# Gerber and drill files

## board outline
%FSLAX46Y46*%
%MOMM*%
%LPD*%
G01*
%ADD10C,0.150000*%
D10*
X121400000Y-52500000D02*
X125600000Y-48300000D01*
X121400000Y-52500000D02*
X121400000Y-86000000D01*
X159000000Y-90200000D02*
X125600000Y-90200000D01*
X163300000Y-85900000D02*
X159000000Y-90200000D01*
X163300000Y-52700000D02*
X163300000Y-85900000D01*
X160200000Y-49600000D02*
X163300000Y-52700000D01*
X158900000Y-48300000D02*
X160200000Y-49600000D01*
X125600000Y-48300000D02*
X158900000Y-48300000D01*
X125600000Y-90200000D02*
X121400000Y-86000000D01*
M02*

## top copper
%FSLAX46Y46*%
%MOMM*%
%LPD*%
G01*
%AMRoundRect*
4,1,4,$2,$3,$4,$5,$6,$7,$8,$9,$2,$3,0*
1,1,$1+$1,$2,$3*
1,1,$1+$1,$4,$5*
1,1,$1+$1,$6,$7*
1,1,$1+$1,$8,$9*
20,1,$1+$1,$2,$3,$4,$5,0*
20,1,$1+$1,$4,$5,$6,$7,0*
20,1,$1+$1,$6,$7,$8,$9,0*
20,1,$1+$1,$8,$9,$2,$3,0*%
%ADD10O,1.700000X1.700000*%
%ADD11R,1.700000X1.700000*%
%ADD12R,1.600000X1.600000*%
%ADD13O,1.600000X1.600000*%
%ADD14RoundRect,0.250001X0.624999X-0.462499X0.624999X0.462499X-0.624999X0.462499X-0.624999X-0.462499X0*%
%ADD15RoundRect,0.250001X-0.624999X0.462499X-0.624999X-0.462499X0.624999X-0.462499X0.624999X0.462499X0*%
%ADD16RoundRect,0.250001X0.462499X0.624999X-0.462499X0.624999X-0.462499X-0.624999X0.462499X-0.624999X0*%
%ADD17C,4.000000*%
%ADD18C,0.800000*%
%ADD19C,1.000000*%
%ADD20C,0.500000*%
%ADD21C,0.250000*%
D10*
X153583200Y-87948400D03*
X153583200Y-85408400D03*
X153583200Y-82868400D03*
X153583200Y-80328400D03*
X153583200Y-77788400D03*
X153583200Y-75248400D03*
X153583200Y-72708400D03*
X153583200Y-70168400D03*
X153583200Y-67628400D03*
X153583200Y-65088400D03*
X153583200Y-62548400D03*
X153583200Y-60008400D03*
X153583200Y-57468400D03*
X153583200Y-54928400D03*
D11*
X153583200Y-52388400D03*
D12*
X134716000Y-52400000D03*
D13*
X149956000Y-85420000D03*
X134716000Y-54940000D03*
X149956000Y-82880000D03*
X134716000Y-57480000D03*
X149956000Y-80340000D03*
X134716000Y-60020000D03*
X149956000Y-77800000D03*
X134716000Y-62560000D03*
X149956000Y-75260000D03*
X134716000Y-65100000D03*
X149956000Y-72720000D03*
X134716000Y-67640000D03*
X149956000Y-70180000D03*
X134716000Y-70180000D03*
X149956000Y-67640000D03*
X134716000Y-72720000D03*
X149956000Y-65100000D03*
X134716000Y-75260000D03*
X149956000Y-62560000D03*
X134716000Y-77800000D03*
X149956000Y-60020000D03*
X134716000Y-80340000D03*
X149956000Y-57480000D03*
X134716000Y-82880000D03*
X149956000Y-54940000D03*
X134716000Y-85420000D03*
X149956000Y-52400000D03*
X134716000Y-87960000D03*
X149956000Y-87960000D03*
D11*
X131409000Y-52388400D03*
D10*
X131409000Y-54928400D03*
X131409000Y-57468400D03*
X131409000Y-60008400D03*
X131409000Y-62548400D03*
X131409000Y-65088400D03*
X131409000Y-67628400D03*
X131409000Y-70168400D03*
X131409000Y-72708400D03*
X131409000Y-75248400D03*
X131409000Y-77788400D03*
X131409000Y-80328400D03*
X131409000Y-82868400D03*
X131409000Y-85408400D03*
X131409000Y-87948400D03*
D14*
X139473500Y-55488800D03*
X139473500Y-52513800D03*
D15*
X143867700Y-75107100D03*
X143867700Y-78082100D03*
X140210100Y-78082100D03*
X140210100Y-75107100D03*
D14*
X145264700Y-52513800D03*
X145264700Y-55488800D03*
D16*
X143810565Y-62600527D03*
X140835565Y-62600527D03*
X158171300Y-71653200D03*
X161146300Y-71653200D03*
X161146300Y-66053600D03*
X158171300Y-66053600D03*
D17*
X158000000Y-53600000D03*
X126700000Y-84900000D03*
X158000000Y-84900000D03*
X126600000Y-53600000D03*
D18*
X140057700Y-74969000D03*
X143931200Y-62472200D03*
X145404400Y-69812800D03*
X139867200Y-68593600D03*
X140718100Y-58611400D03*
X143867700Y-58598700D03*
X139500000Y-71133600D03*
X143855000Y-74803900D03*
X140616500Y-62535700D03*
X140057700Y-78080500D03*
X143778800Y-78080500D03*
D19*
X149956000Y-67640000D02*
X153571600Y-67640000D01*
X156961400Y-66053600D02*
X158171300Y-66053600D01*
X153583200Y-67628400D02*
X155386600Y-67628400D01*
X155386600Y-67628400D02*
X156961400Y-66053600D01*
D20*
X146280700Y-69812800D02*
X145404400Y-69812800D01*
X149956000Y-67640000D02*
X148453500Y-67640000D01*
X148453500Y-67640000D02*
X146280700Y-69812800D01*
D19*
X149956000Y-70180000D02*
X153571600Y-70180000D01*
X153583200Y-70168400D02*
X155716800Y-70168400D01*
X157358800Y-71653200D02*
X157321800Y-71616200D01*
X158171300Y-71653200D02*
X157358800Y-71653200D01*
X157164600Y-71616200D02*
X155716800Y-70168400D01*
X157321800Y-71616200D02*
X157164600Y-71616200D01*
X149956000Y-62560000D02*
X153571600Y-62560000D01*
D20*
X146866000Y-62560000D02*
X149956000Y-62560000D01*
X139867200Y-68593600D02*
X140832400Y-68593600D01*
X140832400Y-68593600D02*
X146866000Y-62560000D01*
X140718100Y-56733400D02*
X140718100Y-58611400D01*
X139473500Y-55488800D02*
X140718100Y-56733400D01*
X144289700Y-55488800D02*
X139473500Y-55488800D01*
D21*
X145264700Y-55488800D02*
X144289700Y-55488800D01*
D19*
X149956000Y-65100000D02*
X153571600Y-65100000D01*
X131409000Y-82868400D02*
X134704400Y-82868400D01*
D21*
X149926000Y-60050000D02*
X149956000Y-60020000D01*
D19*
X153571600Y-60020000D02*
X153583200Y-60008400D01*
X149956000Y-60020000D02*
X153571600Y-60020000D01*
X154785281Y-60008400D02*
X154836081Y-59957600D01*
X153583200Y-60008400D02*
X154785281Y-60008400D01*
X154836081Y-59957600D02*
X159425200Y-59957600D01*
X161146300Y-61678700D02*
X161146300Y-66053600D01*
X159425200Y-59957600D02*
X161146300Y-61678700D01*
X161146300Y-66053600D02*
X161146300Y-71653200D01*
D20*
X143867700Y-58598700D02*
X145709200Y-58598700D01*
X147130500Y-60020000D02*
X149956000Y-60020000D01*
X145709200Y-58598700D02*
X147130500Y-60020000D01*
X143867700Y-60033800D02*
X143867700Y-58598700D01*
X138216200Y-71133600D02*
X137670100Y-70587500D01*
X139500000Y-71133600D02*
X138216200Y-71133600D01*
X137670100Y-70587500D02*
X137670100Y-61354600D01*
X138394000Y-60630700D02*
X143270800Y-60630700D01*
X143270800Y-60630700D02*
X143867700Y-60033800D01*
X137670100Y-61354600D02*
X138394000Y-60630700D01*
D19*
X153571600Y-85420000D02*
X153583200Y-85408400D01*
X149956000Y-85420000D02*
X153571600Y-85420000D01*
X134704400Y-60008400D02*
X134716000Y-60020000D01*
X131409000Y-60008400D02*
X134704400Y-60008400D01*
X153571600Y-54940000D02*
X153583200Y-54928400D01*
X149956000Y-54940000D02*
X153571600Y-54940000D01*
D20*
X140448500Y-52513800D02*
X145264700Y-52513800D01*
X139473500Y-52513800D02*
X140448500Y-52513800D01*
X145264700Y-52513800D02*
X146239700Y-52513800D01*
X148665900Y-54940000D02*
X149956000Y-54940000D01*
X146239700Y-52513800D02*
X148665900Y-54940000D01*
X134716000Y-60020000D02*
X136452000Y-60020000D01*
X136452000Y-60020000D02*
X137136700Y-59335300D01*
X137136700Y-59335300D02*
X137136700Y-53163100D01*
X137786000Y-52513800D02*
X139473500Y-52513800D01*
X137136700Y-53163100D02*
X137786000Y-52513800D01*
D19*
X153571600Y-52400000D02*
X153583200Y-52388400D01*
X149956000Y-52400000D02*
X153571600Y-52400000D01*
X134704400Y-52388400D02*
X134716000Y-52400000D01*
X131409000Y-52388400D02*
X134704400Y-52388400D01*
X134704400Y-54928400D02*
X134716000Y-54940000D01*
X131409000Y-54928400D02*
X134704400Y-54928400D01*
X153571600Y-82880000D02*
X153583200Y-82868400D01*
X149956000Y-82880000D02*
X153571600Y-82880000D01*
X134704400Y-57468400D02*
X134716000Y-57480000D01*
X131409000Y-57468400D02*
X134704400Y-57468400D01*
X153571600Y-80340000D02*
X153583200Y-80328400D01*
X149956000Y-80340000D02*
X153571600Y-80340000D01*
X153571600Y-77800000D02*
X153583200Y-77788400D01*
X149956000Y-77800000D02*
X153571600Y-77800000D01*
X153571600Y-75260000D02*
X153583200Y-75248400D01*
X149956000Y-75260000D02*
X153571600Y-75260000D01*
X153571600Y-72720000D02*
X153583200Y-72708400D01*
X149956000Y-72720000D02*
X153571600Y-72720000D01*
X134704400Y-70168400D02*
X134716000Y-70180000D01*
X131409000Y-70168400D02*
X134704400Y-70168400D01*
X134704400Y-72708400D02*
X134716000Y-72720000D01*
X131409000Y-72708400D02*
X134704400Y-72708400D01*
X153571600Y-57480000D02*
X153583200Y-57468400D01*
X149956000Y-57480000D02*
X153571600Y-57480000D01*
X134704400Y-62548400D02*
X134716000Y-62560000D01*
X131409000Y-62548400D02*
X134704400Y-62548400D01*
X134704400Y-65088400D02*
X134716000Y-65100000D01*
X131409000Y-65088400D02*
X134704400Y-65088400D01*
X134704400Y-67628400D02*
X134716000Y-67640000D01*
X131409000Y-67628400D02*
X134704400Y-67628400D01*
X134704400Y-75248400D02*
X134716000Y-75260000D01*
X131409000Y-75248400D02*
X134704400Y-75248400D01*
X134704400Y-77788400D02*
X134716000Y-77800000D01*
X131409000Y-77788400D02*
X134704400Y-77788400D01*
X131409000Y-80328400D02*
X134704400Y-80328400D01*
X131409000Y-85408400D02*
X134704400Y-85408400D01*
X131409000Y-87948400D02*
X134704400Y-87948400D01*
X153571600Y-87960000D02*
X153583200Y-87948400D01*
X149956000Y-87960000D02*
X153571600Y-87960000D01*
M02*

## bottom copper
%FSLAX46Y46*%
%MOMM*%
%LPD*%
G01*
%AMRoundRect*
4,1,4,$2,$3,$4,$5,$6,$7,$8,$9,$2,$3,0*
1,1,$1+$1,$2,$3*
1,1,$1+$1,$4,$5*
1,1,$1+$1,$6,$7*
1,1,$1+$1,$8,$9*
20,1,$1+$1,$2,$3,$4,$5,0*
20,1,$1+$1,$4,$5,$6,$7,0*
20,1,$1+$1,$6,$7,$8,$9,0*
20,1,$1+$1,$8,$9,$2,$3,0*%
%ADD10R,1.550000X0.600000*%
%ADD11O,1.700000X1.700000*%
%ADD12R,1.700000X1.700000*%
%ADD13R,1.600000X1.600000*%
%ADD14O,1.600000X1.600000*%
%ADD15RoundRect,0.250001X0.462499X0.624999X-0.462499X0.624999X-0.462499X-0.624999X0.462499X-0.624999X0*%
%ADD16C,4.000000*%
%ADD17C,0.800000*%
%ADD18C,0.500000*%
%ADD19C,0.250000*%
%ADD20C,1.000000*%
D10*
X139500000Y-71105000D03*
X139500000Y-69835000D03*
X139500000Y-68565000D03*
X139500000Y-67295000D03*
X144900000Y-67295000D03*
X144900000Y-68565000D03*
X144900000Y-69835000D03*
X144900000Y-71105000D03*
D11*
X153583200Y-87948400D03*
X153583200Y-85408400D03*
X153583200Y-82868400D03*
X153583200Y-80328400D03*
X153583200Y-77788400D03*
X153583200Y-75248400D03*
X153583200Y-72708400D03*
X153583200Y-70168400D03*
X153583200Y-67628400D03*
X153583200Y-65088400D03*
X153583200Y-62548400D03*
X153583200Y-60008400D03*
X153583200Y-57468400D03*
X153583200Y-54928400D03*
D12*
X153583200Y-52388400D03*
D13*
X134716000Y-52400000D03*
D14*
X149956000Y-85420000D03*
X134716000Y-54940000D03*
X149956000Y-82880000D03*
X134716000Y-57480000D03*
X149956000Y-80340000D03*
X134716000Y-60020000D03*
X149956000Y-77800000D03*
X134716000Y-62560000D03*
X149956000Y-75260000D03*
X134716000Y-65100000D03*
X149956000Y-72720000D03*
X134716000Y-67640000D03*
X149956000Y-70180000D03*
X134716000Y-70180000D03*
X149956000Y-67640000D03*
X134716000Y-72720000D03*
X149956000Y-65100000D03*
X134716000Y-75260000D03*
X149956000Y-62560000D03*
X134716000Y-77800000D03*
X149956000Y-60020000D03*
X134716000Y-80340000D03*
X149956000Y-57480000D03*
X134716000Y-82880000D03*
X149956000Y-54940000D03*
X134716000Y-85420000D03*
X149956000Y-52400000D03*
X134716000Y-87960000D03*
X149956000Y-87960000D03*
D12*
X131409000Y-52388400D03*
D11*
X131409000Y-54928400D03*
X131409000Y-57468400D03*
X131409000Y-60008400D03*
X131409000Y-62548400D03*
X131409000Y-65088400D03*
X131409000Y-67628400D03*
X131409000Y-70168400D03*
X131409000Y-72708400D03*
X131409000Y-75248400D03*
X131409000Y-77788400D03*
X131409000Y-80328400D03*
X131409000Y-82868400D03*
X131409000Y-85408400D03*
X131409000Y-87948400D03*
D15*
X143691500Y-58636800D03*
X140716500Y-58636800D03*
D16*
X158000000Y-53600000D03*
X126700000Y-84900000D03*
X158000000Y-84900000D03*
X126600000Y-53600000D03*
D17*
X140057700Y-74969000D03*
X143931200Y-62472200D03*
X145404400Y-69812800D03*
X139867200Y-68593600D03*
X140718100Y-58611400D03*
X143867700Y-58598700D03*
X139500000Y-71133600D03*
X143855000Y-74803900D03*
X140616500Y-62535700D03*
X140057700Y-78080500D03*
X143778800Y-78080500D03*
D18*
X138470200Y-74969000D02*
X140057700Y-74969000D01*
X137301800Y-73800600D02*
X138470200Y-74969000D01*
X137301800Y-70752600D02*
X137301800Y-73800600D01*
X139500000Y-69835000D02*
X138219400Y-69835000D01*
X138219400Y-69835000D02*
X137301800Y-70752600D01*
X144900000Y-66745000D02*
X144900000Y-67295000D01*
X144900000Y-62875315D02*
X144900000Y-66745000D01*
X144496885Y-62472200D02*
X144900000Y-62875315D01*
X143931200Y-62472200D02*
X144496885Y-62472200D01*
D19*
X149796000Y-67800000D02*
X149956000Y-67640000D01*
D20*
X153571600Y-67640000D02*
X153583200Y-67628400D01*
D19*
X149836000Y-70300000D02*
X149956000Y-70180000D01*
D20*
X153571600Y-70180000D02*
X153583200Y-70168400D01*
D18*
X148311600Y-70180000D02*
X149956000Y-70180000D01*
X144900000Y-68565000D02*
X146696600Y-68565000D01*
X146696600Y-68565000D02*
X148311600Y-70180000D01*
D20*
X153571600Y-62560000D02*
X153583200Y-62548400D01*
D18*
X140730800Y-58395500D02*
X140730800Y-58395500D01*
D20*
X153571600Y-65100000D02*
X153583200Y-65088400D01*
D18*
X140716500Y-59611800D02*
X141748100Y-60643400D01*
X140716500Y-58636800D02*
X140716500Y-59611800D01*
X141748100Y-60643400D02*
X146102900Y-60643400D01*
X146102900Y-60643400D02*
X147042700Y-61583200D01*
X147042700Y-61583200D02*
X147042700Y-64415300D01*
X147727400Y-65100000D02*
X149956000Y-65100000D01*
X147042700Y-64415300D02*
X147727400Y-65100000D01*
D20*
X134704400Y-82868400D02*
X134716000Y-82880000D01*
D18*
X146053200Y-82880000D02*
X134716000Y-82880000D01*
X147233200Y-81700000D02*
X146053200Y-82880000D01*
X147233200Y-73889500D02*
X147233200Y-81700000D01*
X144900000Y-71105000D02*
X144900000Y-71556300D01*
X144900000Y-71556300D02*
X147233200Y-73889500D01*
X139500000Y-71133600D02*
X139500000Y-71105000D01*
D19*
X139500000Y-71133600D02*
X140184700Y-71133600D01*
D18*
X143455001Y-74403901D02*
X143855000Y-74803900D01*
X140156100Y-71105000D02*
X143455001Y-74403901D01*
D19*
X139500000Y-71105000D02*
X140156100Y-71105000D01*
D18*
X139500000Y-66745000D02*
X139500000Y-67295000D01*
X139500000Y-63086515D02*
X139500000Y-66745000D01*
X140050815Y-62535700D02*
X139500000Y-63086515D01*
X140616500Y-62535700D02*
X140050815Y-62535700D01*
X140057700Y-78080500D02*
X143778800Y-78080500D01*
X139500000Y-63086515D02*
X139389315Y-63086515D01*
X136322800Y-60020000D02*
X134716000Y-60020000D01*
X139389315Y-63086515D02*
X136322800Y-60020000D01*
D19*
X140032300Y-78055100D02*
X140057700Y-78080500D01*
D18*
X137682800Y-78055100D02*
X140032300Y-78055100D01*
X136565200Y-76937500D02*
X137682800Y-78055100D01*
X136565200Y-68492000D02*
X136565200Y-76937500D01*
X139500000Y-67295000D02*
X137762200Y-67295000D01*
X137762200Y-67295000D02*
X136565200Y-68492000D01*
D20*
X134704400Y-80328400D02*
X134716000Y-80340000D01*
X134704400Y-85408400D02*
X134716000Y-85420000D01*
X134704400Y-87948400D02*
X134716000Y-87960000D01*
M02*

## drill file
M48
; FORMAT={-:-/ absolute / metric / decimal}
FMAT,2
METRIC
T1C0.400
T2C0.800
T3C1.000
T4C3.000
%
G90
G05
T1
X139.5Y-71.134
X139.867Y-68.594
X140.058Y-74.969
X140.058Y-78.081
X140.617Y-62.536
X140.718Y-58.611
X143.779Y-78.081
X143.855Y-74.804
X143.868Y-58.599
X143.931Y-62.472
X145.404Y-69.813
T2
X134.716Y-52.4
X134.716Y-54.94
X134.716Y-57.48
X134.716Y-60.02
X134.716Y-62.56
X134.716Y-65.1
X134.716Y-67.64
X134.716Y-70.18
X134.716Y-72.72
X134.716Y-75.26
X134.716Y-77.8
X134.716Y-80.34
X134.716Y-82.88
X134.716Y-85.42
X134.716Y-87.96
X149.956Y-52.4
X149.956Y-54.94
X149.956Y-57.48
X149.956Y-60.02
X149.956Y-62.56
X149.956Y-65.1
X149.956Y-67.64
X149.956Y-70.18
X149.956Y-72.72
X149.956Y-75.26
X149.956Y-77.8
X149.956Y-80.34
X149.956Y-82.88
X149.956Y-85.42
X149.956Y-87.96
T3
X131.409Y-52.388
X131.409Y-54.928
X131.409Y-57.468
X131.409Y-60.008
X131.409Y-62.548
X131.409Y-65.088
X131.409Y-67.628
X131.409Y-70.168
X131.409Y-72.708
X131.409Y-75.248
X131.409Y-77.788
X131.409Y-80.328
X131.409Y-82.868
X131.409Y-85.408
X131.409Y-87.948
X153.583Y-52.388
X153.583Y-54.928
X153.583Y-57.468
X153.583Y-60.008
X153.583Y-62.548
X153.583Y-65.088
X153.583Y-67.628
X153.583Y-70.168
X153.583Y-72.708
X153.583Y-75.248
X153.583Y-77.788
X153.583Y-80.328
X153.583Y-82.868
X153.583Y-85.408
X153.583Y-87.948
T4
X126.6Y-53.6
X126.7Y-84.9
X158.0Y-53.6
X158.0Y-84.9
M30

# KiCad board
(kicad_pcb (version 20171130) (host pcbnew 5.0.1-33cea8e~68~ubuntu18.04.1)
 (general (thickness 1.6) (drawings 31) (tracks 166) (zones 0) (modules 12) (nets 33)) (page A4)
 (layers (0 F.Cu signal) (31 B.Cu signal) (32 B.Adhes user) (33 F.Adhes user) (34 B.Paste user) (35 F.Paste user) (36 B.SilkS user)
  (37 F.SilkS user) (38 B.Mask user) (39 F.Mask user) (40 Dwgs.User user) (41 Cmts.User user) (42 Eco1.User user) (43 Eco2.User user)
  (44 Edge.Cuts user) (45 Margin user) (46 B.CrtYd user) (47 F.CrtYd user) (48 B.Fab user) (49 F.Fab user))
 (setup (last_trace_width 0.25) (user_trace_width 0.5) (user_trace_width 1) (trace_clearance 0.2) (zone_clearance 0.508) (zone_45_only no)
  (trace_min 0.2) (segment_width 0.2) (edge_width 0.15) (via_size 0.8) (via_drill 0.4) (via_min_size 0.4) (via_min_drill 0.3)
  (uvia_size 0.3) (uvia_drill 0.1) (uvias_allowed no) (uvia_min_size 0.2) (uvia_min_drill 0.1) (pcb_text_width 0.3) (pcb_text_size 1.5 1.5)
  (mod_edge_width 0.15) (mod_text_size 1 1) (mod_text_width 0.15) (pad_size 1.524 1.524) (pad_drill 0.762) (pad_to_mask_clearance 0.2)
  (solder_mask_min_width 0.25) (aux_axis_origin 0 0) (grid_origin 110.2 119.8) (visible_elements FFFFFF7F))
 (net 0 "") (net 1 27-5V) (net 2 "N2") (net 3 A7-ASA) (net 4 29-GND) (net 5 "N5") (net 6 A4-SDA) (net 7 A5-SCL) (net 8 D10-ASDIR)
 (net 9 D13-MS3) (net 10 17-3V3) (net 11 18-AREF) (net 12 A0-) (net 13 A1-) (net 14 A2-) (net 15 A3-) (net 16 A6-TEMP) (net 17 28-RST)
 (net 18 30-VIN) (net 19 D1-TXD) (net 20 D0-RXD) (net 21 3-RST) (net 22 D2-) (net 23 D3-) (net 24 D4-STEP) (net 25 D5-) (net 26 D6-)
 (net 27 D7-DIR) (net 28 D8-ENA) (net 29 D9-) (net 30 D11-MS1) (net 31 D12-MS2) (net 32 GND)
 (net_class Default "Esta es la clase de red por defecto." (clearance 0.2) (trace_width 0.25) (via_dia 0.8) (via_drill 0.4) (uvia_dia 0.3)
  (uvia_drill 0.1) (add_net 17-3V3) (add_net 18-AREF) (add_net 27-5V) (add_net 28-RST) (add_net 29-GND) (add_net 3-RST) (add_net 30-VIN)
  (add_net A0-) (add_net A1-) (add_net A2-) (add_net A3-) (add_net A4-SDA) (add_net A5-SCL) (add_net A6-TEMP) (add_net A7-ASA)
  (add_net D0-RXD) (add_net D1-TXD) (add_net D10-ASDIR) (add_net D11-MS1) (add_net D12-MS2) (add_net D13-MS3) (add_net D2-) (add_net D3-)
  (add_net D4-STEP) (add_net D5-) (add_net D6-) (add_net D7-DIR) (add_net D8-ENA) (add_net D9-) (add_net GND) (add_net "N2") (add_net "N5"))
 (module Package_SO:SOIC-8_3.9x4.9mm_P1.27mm (layer B.Cu) (at 142.2 69.2)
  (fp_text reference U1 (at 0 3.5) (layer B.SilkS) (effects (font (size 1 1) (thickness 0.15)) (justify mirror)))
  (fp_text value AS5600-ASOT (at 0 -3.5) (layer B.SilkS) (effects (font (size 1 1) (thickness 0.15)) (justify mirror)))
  (pad 1 smd rect (at -2.7 1.905) (size 1.55 0.6) (layers B.Cu B.Paste B.Mask) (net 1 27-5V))
  (pad 2 smd rect (at -2.7 0.635) (size 1.55 0.6) (layers B.Cu B.Paste B.Mask) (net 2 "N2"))
  (pad 3 smd rect (at -2.7 -0.635) (size 1.55 0.6) (layers B.Cu B.Paste B.Mask) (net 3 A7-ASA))
  (pad 4 smd rect (at -2.7 -1.905) (size 1.55 0.6) (layers B.Cu B.Paste B.Mask) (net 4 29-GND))
  (pad 5 smd rect (at 2.7 -1.905) (size 1.55 0.6) (layers B.Cu B.Paste B.Mask) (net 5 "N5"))
  (pad 6 smd rect (at 2.7 -0.635) (size 1.55 0.6) (layers B.Cu B.Paste B.Mask) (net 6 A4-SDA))
  (pad 7 smd rect (at 2.7 0.635) (size 1.55 0.6) (layers B.Cu B.Paste B.Mask) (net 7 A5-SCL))
  (pad 8 smd rect (at 2.7 1.905) (size 1.55 0.6) (layers B.Cu B.Paste B.Mask) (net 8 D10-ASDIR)))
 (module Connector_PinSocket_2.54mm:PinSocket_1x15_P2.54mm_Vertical (layer F.Cu) (at 153.5832 52.3884)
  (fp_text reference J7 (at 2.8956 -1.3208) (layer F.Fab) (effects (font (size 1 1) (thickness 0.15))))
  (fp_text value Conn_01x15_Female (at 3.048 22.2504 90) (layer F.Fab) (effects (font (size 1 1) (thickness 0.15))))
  (pad 15 thru_hole oval (at 0 35.56) (size 1.7 1.7) (drill 1) (layers *.Cu *.Mask) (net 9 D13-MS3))
  (pad 14 thru_hole oval (at 0 33.02) (size 1.7 1.7) (drill 1) (layers *.Cu *.Mask) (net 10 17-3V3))
  (pad 13 thru_hole oval (at 0 30.48) (size 1.7 1.7) (drill 1) (layers *.Cu *.Mask) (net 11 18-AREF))
  (pad 12 thru_hole oval (at 0 27.94) (size 1.7 1.7) (drill 1) (layers *.Cu *.Mask) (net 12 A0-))
  (pad 11 thru_hole oval (at 0 25.4) (size 1.7 1.7) (drill 1) (layers *.Cu *.Mask) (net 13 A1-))
  (pad 10 thru_hole oval (at 0 22.86) (size 1.7 1.7) (drill 1) (layers *.Cu *.Mask) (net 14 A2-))
  (pad 9 thru_hole oval (at 0 20.32) (size 1.7 1.7) (drill 1) (layers *.Cu *.Mask) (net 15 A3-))
  (pad 8 thru_hole oval (at 0 17.78) (size 1.7 1.7) (drill 1) (layers *.Cu *.Mask) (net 6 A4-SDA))
  (pad 7 thru_hole oval (at 0 15.24) (size 1.7 1.7) (drill 1) (layers *.Cu *.Mask) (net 7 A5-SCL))
  (pad 6 thru_hole oval (at 0 12.7) (size 1.7 1.7) (drill 1) (layers *.Cu *.Mask) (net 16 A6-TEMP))
  (pad 5 thru_hole oval (at 0 10.16) (size 1.7 1.7) (drill 1) (layers *.Cu *.Mask) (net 3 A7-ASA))
  (pad 4 thru_hole oval (at 0 7.62) (size 1.7 1.7) (drill 1) (layers *.Cu *.Mask) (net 1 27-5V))
  (pad 3 thru_hole oval (at 0 5.08) (size 1.7 1.7) (drill 1) (layers *.Cu *.Mask) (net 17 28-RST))
  (pad 2 thru_hole oval (at 0 2.54) (size 1.7 1.7) (drill 1) (layers *.Cu *.Mask) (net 4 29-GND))
  (pad 1 thru_hole rect (at 0 0) (size 1.7 1.7) (drill 1) (layers *.Cu *.Mask) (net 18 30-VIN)))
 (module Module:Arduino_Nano (layer F.Cu) (at 134.716 52.4)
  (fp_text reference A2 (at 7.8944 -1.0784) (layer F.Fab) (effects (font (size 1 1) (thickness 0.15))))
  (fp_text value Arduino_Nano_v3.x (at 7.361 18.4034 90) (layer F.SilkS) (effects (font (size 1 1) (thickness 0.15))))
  (pad 1 thru_hole rect (at 0 0) (size 1.6 1.6) (drill 0.8) (layers *.Cu *.Mask) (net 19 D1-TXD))
  (pad 17 thru_hole oval (at 15.24 33.02) (size 1.6 1.6) (drill 0.8) (layers *.Cu *.Mask) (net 10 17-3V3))
  (pad 2 thru_hole oval (at 0 2.54) (size 1.6 1.6) (drill 0.8) (layers *.Cu *.Mask) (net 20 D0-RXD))
  (pad 18 thru_hole oval (at 15.24 30.48) (size 1.6 1.6) (drill 0.8) (layers *.Cu *.Mask) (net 11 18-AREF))
  (pad 3 thru_hole oval (at 0 5.08) (size 1.6 1.6) (drill 0.8) (layers *.Cu *.Mask) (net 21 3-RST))
  (pad 19 thru_hole oval (at 15.24 27.94) (size 1.6 1.6) (drill 0.8) (layers *.Cu *.Mask) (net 12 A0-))
  (pad 4 thru_hole oval (at 0 7.62) (size 1.6 1.6) (drill 0.8) (layers *.Cu *.Mask) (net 4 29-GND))
  (pad 20 thru_hole oval (at 15.24 25.4) (size 1.6 1.6) (drill 0.8) (layers *.Cu *.Mask) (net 13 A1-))
  (pad 5 thru_hole oval (at 0 10.16) (size 1.6 1.6) (drill 0.8) (layers *.Cu *.Mask) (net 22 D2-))
  (pad 21 thru_hole oval (at 15.24 22.86) (size 1.6 1.6) (drill 0.8) (layers *.Cu *.Mask) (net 14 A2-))
  (pad 6 thru_hole oval (at 0 12.7) (size 1.6 1.6) (drill 0.8) (layers *.Cu *.Mask) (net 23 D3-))
  (pad 22 thru_hole oval (at 15.24 20.32) (size 1.6 1.6) (drill 0.8) (layers *.Cu *.Mask) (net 15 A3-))
  (pad 7 thru_hole oval (at 0 15.24) (size 1.6 1.6) (drill 0.8) (layers *.Cu *.Mask) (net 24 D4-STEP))
  (pad 23 thru_hole oval (at 15.24 17.78) (size 1.6 1.6) (drill 0.8) (layers *.Cu *.Mask) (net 6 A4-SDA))
  (pad 8 thru_hole oval (at 0 17.78) (size 1.6 1.6) (drill 0.8) (layers *.Cu *.Mask) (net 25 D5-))
  (pad 24 thru_hole oval (at 15.24 15.24) (size 1.6 1.6) (drill 0.8) (layers *.Cu *.Mask) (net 7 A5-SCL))
  (pad 9 thru_hole oval (at 0 20.32) (size 1.6 1.6) (drill 0.8) (layers *.Cu *.Mask) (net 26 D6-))
  (pad 25 thru_hole oval (at 15.24 12.7) (size 1.6 1.6) (drill 0.8) (layers *.Cu *.Mask) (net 16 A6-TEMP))
  (pad 10 thru_hole oval (at 0 22.86) (size 1.6 1.6) (drill 0.8) (layers *.Cu *.Mask) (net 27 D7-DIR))
  (pad 26 thru_hole oval (at 15.24 10.16) (size 1.6 1.6) (drill 0.8) (layers *.Cu *.Mask) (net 3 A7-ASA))
  (pad 11 thru_hole oval (at 0 25.4) (size 1.6 1.6) (drill 0.8) (layers *.Cu *.Mask) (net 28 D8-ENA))
  (pad 27 thru_hole oval (at 15.24 7.62) (size 1.6 1.6) (drill 0.8) (layers *.Cu *.Mask) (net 1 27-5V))
  (pad 12 thru_hole oval (at 0 27.94) (size 1.6 1.6) (drill 0.8) (layers *.Cu *.Mask) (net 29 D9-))
  (pad 28 thru_hole oval (at 15.24 5.08) (size 1.6 1.6) (drill 0.8) (layers *.Cu *.Mask) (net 17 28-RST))
  (pad 13 thru_hole oval (at 0 30.48) (size 1.6 1.6) (drill 0.8) (layers *.Cu *.Mask) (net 8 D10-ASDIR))
  (pad 29 thru_hole oval (at 15.24 2.54) (size 1.6 1.6) (drill 0.8) (layers *.Cu *.Mask) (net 4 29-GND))
  (pad 14 thru_hole oval (at 0 33.02) (size 1.6 1.6) (drill 0.8) (layers *.Cu *.Mask) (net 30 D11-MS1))
  (pad 30 thru_hole oval (at 15.24 0) (size 1.6 1.6) (drill 0.8) (layers *.Cu *.Mask) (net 18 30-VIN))
  (pad 15 thru_hole oval (at 0 35.56) (size 1.6 1.6) (drill 0.8) (layers *.Cu *.Mask) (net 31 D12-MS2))
  (pad 16 thru_hole oval (at 15.24 35.56) (size 1.6 1.6) (drill 0.8) (layers *.Cu *.Mask) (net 9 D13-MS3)))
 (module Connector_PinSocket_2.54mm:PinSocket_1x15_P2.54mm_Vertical (layer F.Cu) (at 131.409 52.3884)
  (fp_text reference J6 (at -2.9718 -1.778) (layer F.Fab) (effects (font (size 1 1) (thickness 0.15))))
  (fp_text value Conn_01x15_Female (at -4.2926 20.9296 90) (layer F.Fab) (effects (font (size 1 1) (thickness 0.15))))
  (pad 1 thru_hole rect (at 0 0) (size 1.7 1.7) (drill 1) (layers *.Cu *.Mask) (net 19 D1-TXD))
  (pad 2 thru_hole oval (at 0 2.54) (size 1.7 1.7) (drill 1) (layers *.Cu *.Mask) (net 20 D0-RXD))
  (pad 3 thru_hole oval (at 0 5.08) (size 1.7 1.7) (drill 1) (layers *.Cu *.Mask) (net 21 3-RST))
  (pad 4 thru_hole oval (at 0 7.62) (size 1.7 1.7) (drill 1) (layers *.Cu *.Mask) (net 4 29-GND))
  (pad 5 thru_hole oval (at 0 10.16) (size 1.7 1.7) (drill 1) (layers *.Cu *.Mask) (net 22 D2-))
  (pad 6 thru_hole oval (at 0 12.7) (size 1.7 1.7) (drill 1) (layers *.Cu *.Mask) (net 23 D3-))
  (pad 7 thru_hole oval (at 0 15.24) (size 1.7 1.7) (drill 1) (layers *.Cu *.Mask) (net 24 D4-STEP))
  (pad 8 thru_hole oval (at 0 17.78) (size 1.7 1.7) (drill 1) (layers *.Cu *.Mask) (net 25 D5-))
  (pad 9 thru_hole oval (at 0 20.32) (size 1.7 1.7) (drill 1) (layers *.Cu *.Mask) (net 26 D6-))
  (pad 10 thru_hole oval (at 0 22.86) (size 1.7 1.7) (drill 1) (layers *.Cu *.Mask) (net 27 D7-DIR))
  (pad 11 thru_hole oval (at 0 25.4) (size 1.7 1.7) (drill 1) (layers *.Cu *.Mask) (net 28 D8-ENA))
  (pad 12 thru_hole oval (at 0 27.94) (size 1.7 1.7) (drill 1) (layers *.Cu *.Mask) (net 29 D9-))
  (pad 13 thru_hole oval (at 0 30.48) (size 1.7 1.7) (drill 1) (layers *.Cu *.Mask) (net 8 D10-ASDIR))
  (pad 14 thru_hole oval (at 0 33.02) (size 1.7 1.7) (drill 1) (layers *.Cu *.Mask) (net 30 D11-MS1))
  (pad 15 thru_hole oval (at 0 35.56) (size 1.7 1.7) (drill 1) (layers *.Cu *.Mask) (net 31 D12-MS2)))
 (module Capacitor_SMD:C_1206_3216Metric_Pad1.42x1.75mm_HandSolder (layer F.Cu) (at 139.4735 54.0013 90)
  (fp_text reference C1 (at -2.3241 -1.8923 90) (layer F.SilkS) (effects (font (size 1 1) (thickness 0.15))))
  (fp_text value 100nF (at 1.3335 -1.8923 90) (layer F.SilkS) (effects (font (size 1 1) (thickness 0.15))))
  (pad 1 smd roundrect (at -1.4875 0 90) (size 1.425 1.75) (layers F.Cu F.Paste F.Mask) (roundrect_rratio 0.175439) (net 16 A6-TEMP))
  (pad 2 smd roundrect (at 1.4875 0 90) (size 1.425 1.75) (layers F.Cu F.Paste F.Mask) (roundrect_rratio 0.175439) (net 4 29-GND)))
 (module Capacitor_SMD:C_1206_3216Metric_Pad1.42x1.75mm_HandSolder (layer F.Cu) (at 143.8677 76.5946 270)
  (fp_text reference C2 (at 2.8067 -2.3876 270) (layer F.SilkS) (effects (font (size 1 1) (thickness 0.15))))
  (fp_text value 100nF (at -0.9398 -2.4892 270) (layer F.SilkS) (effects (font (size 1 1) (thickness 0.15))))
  (pad 1 smd roundrect (at -1.4875 0 270) (size 1.425 1.75) (layers F.Cu F.Paste F.Mask) (roundrect_rratio 0.175439) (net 1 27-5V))
  (pad 2 smd roundrect (at 1.4875 0 270) (size 1.425 1.75) (layers F.Cu F.Paste F.Mask) (roundrect_rratio 0.175439) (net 4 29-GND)))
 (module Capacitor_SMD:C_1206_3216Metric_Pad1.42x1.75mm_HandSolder (layer F.Cu) (at 140.2101 76.5946 270)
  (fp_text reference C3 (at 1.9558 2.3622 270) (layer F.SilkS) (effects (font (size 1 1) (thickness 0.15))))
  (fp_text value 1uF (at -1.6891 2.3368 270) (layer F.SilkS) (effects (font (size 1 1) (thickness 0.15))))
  (pad 2 smd roundrect (at 1.4875 0 270) (size 1.425 1.75) (layers F.Cu F.Paste F.Mask) (roundrect_rratio 0.175439) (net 4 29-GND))
  (pad 1 smd roundrect (at -1.4875 0 270) (size 1.425 1.75) (layers F.Cu F.Paste F.Mask) (roundrect_rratio 0.175439) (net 2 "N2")))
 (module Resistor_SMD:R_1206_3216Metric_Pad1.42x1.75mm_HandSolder (layer F.Cu) (at 145.2647 54.0013 90)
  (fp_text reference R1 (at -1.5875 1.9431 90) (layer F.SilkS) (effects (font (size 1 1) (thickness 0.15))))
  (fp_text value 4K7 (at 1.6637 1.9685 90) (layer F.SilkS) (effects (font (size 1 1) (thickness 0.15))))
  (pad 2 smd roundrect (at 1.4875 0 90) (size 1.425 1.75) (layers F.Cu F.Paste F.Mask) (roundrect_rratio 0.175439) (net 4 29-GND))
  (pad 1 smd roundrect (at -1.4875 0 90) (size 1.425 1.75) (layers F.Cu F.Paste F.Mask) (roundrect_rratio 0.175439) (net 16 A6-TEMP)))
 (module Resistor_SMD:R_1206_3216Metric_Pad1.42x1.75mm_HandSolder (layer F.Cu) (at 142.323065 62.600527 180)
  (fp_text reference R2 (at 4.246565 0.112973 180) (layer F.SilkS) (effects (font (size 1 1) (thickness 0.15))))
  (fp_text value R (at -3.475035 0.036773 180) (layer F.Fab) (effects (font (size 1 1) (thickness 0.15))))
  (pad 1 smd roundrect (at -1.4875 0 180) (size 1.425 1.75) (layers F.Cu F.Paste F.Mask) (roundrect_rratio 0.175439) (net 5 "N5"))
  (pad 2 smd roundrect (at 1.4875 0 180) (size 1.425 1.75) (layers F.Cu F.Paste F.Mask) (roundrect_rratio 0.175439) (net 4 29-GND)))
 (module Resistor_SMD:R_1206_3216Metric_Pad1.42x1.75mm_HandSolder (layer F.Cu) (at 159.6588 71.6532 180)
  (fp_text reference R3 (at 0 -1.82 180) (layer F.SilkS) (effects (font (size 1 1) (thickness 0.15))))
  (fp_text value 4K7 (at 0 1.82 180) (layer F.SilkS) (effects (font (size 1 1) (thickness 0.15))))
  (pad 2 smd roundrect (at 1.4875 0 180) (size 1.425 1.75) (layers F.Cu F.Paste F.Mask) (roundrect_rratio 0.175439) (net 6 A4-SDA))
  (pad 1 smd roundrect (at -1.4875 0 180) (size 1.425 1.75) (layers F.Cu F.Paste F.Mask) (roundrect_rratio 0.175439) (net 1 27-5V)))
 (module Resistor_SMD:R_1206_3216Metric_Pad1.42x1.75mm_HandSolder (layer F.Cu) (at 159.6588 66.0536 180)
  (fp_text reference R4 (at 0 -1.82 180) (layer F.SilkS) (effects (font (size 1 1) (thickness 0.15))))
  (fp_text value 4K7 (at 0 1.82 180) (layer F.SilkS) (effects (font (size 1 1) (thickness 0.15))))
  (pad 1 smd roundrect (at -1.4875 0 180) (size 1.425 1.75) (layers F.Cu F.Paste F.Mask) (roundrect_rratio 0.175439) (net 1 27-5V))
  (pad 2 smd roundrect (at 1.4875 0 180) (size 1.425 1.75) (layers F.Cu F.Paste F.Mask) (roundrect_rratio 0.175439) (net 7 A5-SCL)))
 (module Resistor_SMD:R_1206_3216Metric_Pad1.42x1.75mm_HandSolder (layer B.Cu) (at 142.204 58.6368 180)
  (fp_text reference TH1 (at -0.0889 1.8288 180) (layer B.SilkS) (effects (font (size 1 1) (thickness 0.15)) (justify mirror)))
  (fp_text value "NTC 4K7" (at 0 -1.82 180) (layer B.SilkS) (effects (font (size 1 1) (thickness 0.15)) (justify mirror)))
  (pad 1 smd roundrect (at -1.4875 0 180) (size 1.425 1.75) (layers B.Cu B.Paste B.Mask) (roundrect_rratio 0.175439) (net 1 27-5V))
  (pad 2 smd roundrect (at 1.4875 0 180) (size 1.425 1.75) (layers B.Cu B.Paste B.Mask) (roundrect_rratio 0.175439) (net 16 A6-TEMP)))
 (gr_line (start 121.4 52.5) (end 125.6 48.3) (layer Edge.Cuts) (width 0.15))
 (gr_line (start 121.4 52.5) (end 121.4 86) (layer Edge.Cuts) (width 0.15))
 (gr_line (start 159 90.2) (end 125.6 90.2) (layer Edge.Cuts) (width 0.15))
 (gr_line (start 163.3 85.9) (end 159 90.2) (layer Edge.Cuts) (width 0.15))
 (gr_line (start 163.3 52.7) (end 163.3 85.9) (layer Edge.Cuts) (width 0.15))
 (gr_line (start 160.2 49.6) (end 163.3 52.7) (layer Edge.Cuts) (width 0.15))
 (gr_line (start 158.9 48.3) (end 160.2 49.6) (layer Edge.Cuts) (width 0.15))
 (gr_line (start 125.6 48.3) (end 158.9 48.3) (layer Edge.Cuts) (width 0.15))
 (gr_line (start 125.6 90.2) (end 121.4 86) (layer Edge.Cuts) (width 0.15))
 (via (at 158 53.6) (size 4) (drill 3) (layers F.Cu B.Cu) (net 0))
 (via (at 126.7 84.9) (size 4) (drill 3) (layers F.Cu B.Cu) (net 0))
 (via (at 158 84.9) (size 4) (drill 3) (layers F.Cu B.Cu) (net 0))
 (via (at 126.6 53.6) (size 4) (drill 3) (layers F.Cu B.Cu) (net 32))
 (via (at 140.0577 74.969) (size 0.8) (drill 0.4) (layers F.Cu B.Cu) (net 2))
 (segment (start 138.4702 74.969) (end 140.0577 74.969) (width 0.5) (layer B.Cu) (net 2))
 (segment (start 137.3018 73.8006) (end 138.4702 74.969) (width 0.5) (layer B.Cu) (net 2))
 (segment (start 137.3018 70.7526) (end 137.3018 73.8006) (width 0.5) (layer B.Cu) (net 2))
 (segment (start 139.5 69.835) (end 138.2194 69.835) (width 0.5) (layer B.Cu) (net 2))
 (segment (start 138.2194 69.835) (end 137.3018 70.7526) (width 0.5) (layer B.Cu) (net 2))
 (via (at 143.9312 62.4722) (size 0.8) (drill 0.4) (layers F.Cu B.Cu) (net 5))
 (segment (start 144.9 66.745) (end 144.9 67.295) (width 0.5) (layer B.Cu) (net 5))
 (segment (start 144.9 62.875315) (end 144.9 66.745) (width 0.5) (layer B.Cu) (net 5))
 (segment (start 144.496885 62.4722) (end 144.9 62.875315) (width 0.5) (layer B.Cu) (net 5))
 (segment (start 143.9312 62.4722) (end 144.496885 62.4722) (width 0.5) (layer B.Cu) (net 5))
 (via (at 145.4044 69.8128) (size 0.8) (drill 0.4) (layers F.Cu B.Cu) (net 7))
 (segment (start 149.796 67.8) (end 149.956 67.64) (width 0.25) (layer B.Cu) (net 7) (status C00030))
 (segment (start 153.5716 67.64) (end 153.5832 67.6284) (width 1) (layer B.Cu) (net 7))
 (segment (start 149.956 67.64) (end 153.5716 67.64) (width 1) (layer F.Cu) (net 7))
 (segment (start 156.9614 66.0536) (end 158.1713 66.0536) (width 1) (layer F.Cu) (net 7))
 (segment (start 153.5832 67.6284) (end 155.3866 67.6284) (width 1) (layer F.Cu) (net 7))
 (segment (start 155.3866 67.6284) (end 156.9614 66.0536) (width 1) (layer F.Cu) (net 7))
 (segment (start 146.2807 69.8128) (end 145.4044 69.8128) (width 0.5) (layer F.Cu) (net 7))
 (segment (start 149.956 67.64) (end 148.4535 67.64) (width 0.5) (layer F.Cu) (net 7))
 (segment (start 148.4535 67.64) (end 146.2807 69.8128) (width 0.5) (layer F.Cu) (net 7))
 (segment (start 149.836 70.3) (end 149.956 70.18) (width 0.25) (layer B.Cu) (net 6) (status C00030))
 (segment (start 153.5716 70.18) (end 153.5832 70.1684) (width 1) (layer B.Cu) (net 6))
 (segment (start 149.956 70.18) (end 153.5716 70.18) (width 1) (layer F.Cu) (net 6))
 (segment (start 153.5832 70.1684) (end 155.7168 70.1684) (width 1) (layer F.Cu) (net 6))
 (segment (start 148.3116 70.18) (end 149.956 70.18) (width 0.5) (layer B.Cu) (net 6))
 (segment (start 144.9 68.565) (end 146.6966 68.565) (width 0.5) (layer B.Cu) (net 6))
 (segment (start 146.6966 68.565) (end 148.3116 70.18) (width 0.5) (layer B.Cu) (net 6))
 (segment (start 157.3588 71.6532) (end 157.3218 71.6162) (width 1) (layer F.Cu) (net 6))
 (segment (start 158.1713 71.6532) (end 157.3588 71.6532) (width 1) (layer F.Cu) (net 6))
 (segment (start 157.1646 71.6162) (end 155.7168 70.1684) (width 1) (layer F.Cu) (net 6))
 (segment (start 157.3218 71.6162) (end 157.1646 71.6162) (width 1) (layer F.Cu) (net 6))
 (via (at 139.8672 68.5936) (size 0.8) (drill 0.4) (layers F.Cu B.Cu) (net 3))
 (segment (start 153.5716 62.56) (end 153.5832 62.5484) (width 1) (layer B.Cu) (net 3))
 (segment (start 149.956 62.56) (end 153.5716 62.56) (width 1) (layer F.Cu) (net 3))
 (segment (start 146.866 62.56) (end 149.956 62.56) (width 0.5) (layer F.Cu) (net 3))
 (segment (start 139.8672 68.5936) (end 140.8324 68.5936) (width 0.5) (layer F.Cu) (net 3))
 (segment (start 140.8324 68.5936) (end 146.866 62.56) (width 0.5) (layer F.Cu) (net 3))
 (segment (start 140.7308 58.3955) (end 140.7308 58.3955) (width 0.5) (layer B.Cu) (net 16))
 (via (at 140.7181 58.6114) (size 0.8) (drill 0.4) (layers F.Cu B.Cu) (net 16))
 (segment (start 140.7181 56.7334) (end 140.7181 58.6114) (width 0.5) (layer F.Cu) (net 16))
 (segment (start 139.4735 55.4888) (end 140.7181 56.7334) (width 0.5) (layer F.Cu) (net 16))
 (segment (start 144.2897 55.4888) (end 139.4735 55.4888) (width 0.5) (layer F.Cu) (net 16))
 (segment (start 145.2647 55.4888) (end 144.2897 55.4888) (width 0.25) (layer F.Cu) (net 16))
 (segment (start 153.5716 65.1) (end 153.5832 65.0884) (width 1) (layer B.Cu) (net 16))
 (segment (start 149.956 65.1) (end 153.5716 65.1) (width 1) (layer F.Cu) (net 16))
 (segment (start 140.7165 59.6118) (end 141.7481 60.6434) (width 0.5) (layer B.Cu) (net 16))
 (segment (start 140.7165 58.6368) (end 140.7165 59.6118) (width 0.5) (layer B.Cu) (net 16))
 (segment (start 141.7481 60.6434) (end 146.1029 60.6434) (width 0.5) (layer B.Cu) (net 16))
 (segment (start 146.1029 60.6434) (end 147.0427 61.5832) (width 0.5) (layer B.Cu) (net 16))
 (segment (start 147.0427 61.5832) (end 147.0427 64.4153) (width 0.5) (layer B.Cu) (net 16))
 (segment (start 147.7274 65.1) (end 149.956 65.1) (width 0.5) (layer B.Cu) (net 16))
 (segment (start 147.0427 64.4153) (end 147.7274 65.1) (width 0.5) (layer B.Cu) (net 16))
 (segment (start 134.7044 82.8684) (end 134.716 82.88) (width 1) (layer B.Cu) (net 8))
 (segment (start 131.409 82.8684) (end 134.7044 82.8684) (width 1) (layer F.Cu) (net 8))
 (segment (start 146.0532 82.88) (end 134.716 82.88) (width 0.5) (layer B.Cu) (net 8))
 (segment (start 147.2332 81.7) (end 146.0532 82.88) (width 0.5) (layer B.Cu) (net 8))
 (segment (start 147.2332 73.8895) (end 147.2332 81.7) (width 0.5) (layer B.Cu) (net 8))
 (segment (start 144.9 71.105) (end 144.9 71.5563) (width 0.5) (layer B.Cu) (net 8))
 (segment (start 144.9 71.5563) (end 147.2332 73.8895) (width 0.5) (layer B.Cu) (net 8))
 (via (at 143.8677 58.5987) (size 0.8) (drill 0.4) (layers F.Cu B.Cu) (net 1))
 (segment (start 149.926 60.05) (end 149.956 60.02) (width 0.25) (layer F.Cu) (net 1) (status 30))
 (segment (start 153.5716 60.02) (end 153.5832 60.0084) (width 1) (layer F.Cu) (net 1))
 (segment (start 149.956 60.02) (end 153.5716 60.02) (width 1) (layer F.Cu) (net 1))
 (segment (start 139.5 71.1336) (end 139.5 71.105) (width 0.5) (layer B.Cu) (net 1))
 (via (at 139.5 71.1336) (size 0.8) (drill 0.4) (layers F.Cu B.Cu) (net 1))
 (segment (start 154.785281 60.0084) (end 154.836081 59.9576) (width 1) (layer F.Cu) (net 1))
 (segment (start 153.5832 60.0084) (end 154.785281 60.0084) (width 1) (layer F.Cu) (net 1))
 (segment (start 154.836081 59.9576) (end 159.4252 59.9576) (width 1) (layer F.Cu) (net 1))
 (segment (start 161.1463 61.6787) (end 161.1463 66.0536) (width 1) (layer F.Cu) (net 1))
 (segment (start 159.4252 59.9576) (end 161.1463 61.6787) (width 1) (layer F.Cu) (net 1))
 (segment (start 161.1463 66.0536) (end 161.1463 71.6532) (width 1) (layer F.Cu) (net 1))
 (segment (start 143.8677 58.5987) (end 145.7092 58.5987) (width 0.5) (layer F.Cu) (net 1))
 (segment (start 147.1305 60.02) (end 149.956 60.02) (width 0.5) (layer F.Cu) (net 1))
 (segment (start 145.7092 58.5987) (end 147.1305 60.02) (width 0.5) (layer F.Cu) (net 1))
 (via (at 143.855 74.8039) (size 0.8) (drill 0.4) (layers F.Cu B.Cu) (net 1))
 (segment (start 139.5 71.1336) (end 140.1847 71.1336) (width 0.25) (layer B.Cu) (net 1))
 (segment (start 143.455001 74.403901) (end 143.855 74.8039) (width 0.5) (layer B.Cu) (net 1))
 (segment (start 140.1561 71.105) (end 143.455001 74.403901) (width 0.5) (layer B.Cu) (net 1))
 (segment (start 139.5 71.105) (end 140.1561 71.105) (width 0.25) (layer B.Cu) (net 1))
 (segment (start 143.8677 60.0338) (end 143.8677 58.5987) (width 0.5) (layer F.Cu) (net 1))
 (segment (start 138.2162 71.1336) (end 137.6701 70.5875) (width 0.5) (layer F.Cu) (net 1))
 (segment (start 139.5 71.1336) (end 138.2162 71.1336) (width 0.5) (layer F.Cu) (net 1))
 (segment (start 137.6701 70.5875) (end 137.6701 61.3546) (width 0.5) (layer F.Cu) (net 1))
 (segment (start 138.394 60.6307) (end 143.2708 60.6307) (width 0.5) (layer F.Cu) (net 1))
 (segment (start 143.2708 60.6307) (end 143.8677 60.0338) (width 0.5) (layer F.Cu) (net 1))
 (segment (start 137.6701 61.3546) (end 138.394 60.6307) (width 0.5) (layer F.Cu) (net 1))
 (segment (start 153.5716 85.42) (end 153.5832 85.4084) (width 1) (layer F.Cu) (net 10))
 (segment (start 149.956 85.42) (end 153.5716 85.42) (width 1) (layer F.Cu) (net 10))
 (via (at 140.6165 62.5357) (size 0.8) (drill 0.4) (layers F.Cu B.Cu) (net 4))
 (segment (start 134.7044 60.0084) (end 134.716 60.02) (width 1) (layer F.Cu) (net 4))
 (segment (start 131.409 60.0084) (end 134.7044 60.0084) (width 1) (layer F.Cu) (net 4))
 (segment (start 153.5716 54.94) (end 153.5832 54.9284) (width 1) (layer F.Cu) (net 4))
 (segment (start 149.956 54.94) (end 153.5716 54.94) (width 1) (layer F.Cu) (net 4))
 (segment (start 139.5 66.745) (end 139.5 67.295) (width 0.5) (layer B.Cu) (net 4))
 (segment (start 139.5 63.086515) (end 139.5 66.745) (width 0.5) (layer B.Cu) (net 4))
 (segment (start 140.050815 62.5357) (end 139.5 63.086515) (width 0.5) (layer B.Cu) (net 4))
 (segment (start 140.6165 62.5357) (end 140.050815 62.5357) (width 0.5) (layer B.Cu) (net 4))
 (segment (start 140.4485 52.5138) (end 145.2647 52.5138) (width 0.5) (layer F.Cu) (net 4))
 (segment (start 139.4735 52.5138) (end 140.4485 52.5138) (width 0.5) (layer F.Cu) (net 4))
 (segment (start 145.2647 52.5138) (end 146.2397 52.5138) (width 0.5) (layer F.Cu) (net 4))
 (segment (start 148.6659 54.94) (end 149.956 54.94) (width 0.5) (layer F.Cu) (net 4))
 (segment (start 146.2397 52.5138) (end 148.6659 54.94) (width 0.5) (layer F.Cu) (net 4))
 (segment (start 134.716 60.02) (end 136.452 60.02) (width 0.5) (layer F.Cu) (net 4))
 (segment (start 136.452 60.02) (end 137.1367 59.3353) (width 0.5) (layer F.Cu) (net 4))
 (segment (start 137.1367 59.3353) (end 137.1367 53.1631) (width 0.5) (layer F.Cu) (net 4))
 (segment (start 137.786 52.5138) (end 139.4735 52.5138) (width 0.5) (layer F.Cu) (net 4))
 (segment (start 137.1367 53.1631) (end 137.786 52.5138) (width 0.5) (layer F.Cu) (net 4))
 (via (at 140.0577 78.0805) (size 0.8) (drill 0.4) (layers F.Cu B.Cu) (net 4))
 (via (at 143.7788 78.0805) (size 0.8) (drill 0.4) (layers F.Cu B.Cu) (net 4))
 (segment (start 140.0577 78.0805) (end 143.7788 78.0805) (width 0.5) (layer B.Cu) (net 4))
 (segment (start 139.5 63.086515) (end 139.389315 63.086515) (width 0.5) (layer B.Cu) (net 4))
 (segment (start 136.3228 60.02) (end 134.716 60.02) (width 0.5) (layer B.Cu) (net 4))
 (segment (start 139.389315 63.086515) (end 136.3228 60.02) (width 0.5) (layer B.Cu) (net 4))
 (segment (start 140.0323 78.0551) (end 140.0577 78.0805) (width 0.25) (layer B.Cu) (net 4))
 (segment (start 137.6828 78.0551) (end 140.0323 78.0551) (width 0.5) (layer B.Cu) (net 4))
 (segment (start 136.5652 76.9375) (end 137.6828 78.0551) (width 0.5) (layer B.Cu) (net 4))
 (segment (start 136.5652 68.492) (end 136.5652 76.9375) (width 0.5) (layer B.Cu) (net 4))
 (segment (start 139.5 67.295) (end 137.7622 67.295) (width 0.5) (layer B.Cu) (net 4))
 (segment (start 137.7622 67.295) (end 136.5652 68.492) (width 0.5) (layer B.Cu) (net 4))
 (segment (start 153.5716 52.4) (end 153.5832 52.3884) (width 1) (layer F.Cu) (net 18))
 (segment (start 149.956 52.4) (end 153.5716 52.4) (width 1) (layer F.Cu) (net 18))
 (segment (start 134.7044 52.3884) (end 134.716 52.4) (width 1) (layer F.Cu) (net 19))
 (segment (start 131.409 52.3884) (end 134.7044 52.3884) (width 1) (layer F.Cu) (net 19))
 (segment (start 134.7044 54.9284) (end 134.716 54.94) (width 1) (layer F.Cu) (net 20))
 (segment (start 131.409 54.9284) (end 134.7044 54.9284) (width 1) (layer F.Cu) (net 20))
 (segment (start 153.5716 82.88) (end 153.5832 82.8684) (width 1) (layer F.Cu) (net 11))
 (segment (start 149.956 82.88) (end 153.5716 82.88) (width 1) (layer F.Cu) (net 11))
 (segment (start 134.7044 57.4684) (end 134.716 57.48) (width 1) (layer F.Cu) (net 21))
 (segment (start 131.409 57.4684) (end 134.7044 57.4684) (width 1) (layer F.Cu) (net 21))
 (segment (start 153.5716 80.34) (end 153.5832 80.3284) (width 1) (layer F.Cu) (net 12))
 (segment (start 149.956 80.34) (end 153.5716 80.34) (width 1) (layer F.Cu) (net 12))
 (segment (start 153.5716 77.8) (end 153.5832 77.7884) (width 1) (layer F.Cu) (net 13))
 (segment (start 149.956 77.8) (end 153.5716 77.8) (width 1) (layer F.Cu) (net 13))
 (segment (start 153.5716 75.26) (end 153.5832 75.2484) (width 1) (layer F.Cu) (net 14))
 (segment (start 149.956 75.26) (end 153.5716 75.26) (width 1) (layer F.Cu) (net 14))
 (segment (start 153.5716 72.72) (end 153.5832 72.7084) (width 1) (layer F.Cu) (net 15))
 (segment (start 149.956 72.72) (end 153.5716 72.72) (width 1) (layer F.Cu) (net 15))
 (segment (start 134.7044 70.1684) (end 134.716 70.18) (width 1) (layer F.Cu) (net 25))
 (segment (start 131.409 70.1684) (end 134.7044 70.1684) (width 1) (layer F.Cu) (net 25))
 (segment (start 134.7044 72.7084) (end 134.716 72.72) (width 1) (layer F.Cu) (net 26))
 (segment (start 131.409 72.7084) (end 134.7044 72.7084) (width 1) (layer F.Cu) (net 26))
 (segment (start 153.5716 57.48) (end 153.5832 57.4684) (width 1) (layer F.Cu) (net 17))
 (segment (start 149.956 57.48) (end 153.5716 57.48) (width 1) (layer F.Cu) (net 17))
 (segment (start 134.7044 62.5484) (end 134.716 62.56) (width 1) (layer F.Cu) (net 22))
 (segment (start 131.409 62.5484) (end 134.7044 62.5484) (width 1) (layer F.Cu) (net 22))
 (segment (start 134.7044 65.0884) (end 134.716 65.1) (width 1) (layer F.Cu) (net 23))
 (segment (start 131.409 65.0884) (end 134.7044 65.0884) (width 1) (layer F.Cu) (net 23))
 (segment (start 134.7044 67.6284) (end 134.716 67.64) (width 1) (layer F.Cu) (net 24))
 (segment (start 131.409 67.6284) (end 134.7044 67.6284) (width 1) (layer F.Cu) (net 24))
 (segment (start 134.7044 75.2484) (end 134.716 75.26) (width 1) (layer F.Cu) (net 27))
 (segment (start 131.409 75.2484) (end 134.7044 75.2484) (width 1) (layer F.Cu) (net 27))
 (segment (start 134.7044 77.7884) (end 134.716 77.8) (width 1) (layer F.Cu) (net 28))
 (segment (start 131.409 77.7884) (end 134.7044 77.7884) (width 1) (layer F.Cu) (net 28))
 (segment (start 134.7044 80.3284) (end 134.716 80.34) (width 1) (layer B.Cu) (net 29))
 (segment (start 131.409 80.3284) (end 134.7044 80.3284) (width 1) (layer F.Cu) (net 29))
 (segment (start 134.7044 85.4084) (end 134.716 85.42) (width 1) (layer B.Cu) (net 30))
 (segment (start 131.409 85.4084) (end 134.7044 85.4084) (width 1) (layer F.Cu) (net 30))
 (segment (start 134.7044 87.9484) (end 134.716 87.96) (width 1) (layer B.Cu) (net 31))
 (segment (start 131.409 87.9484) (end 134.7044 87.9484) (width 1) (layer F.Cu) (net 31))
 (segment (start 153.5716 87.96) (end 153.5832 87.9484) (width 1) (layer F.Cu) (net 9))
 (segment (start 149.956 87.96) (end 153.5716 87.96) (width 1) (layer F.Cu) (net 9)))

